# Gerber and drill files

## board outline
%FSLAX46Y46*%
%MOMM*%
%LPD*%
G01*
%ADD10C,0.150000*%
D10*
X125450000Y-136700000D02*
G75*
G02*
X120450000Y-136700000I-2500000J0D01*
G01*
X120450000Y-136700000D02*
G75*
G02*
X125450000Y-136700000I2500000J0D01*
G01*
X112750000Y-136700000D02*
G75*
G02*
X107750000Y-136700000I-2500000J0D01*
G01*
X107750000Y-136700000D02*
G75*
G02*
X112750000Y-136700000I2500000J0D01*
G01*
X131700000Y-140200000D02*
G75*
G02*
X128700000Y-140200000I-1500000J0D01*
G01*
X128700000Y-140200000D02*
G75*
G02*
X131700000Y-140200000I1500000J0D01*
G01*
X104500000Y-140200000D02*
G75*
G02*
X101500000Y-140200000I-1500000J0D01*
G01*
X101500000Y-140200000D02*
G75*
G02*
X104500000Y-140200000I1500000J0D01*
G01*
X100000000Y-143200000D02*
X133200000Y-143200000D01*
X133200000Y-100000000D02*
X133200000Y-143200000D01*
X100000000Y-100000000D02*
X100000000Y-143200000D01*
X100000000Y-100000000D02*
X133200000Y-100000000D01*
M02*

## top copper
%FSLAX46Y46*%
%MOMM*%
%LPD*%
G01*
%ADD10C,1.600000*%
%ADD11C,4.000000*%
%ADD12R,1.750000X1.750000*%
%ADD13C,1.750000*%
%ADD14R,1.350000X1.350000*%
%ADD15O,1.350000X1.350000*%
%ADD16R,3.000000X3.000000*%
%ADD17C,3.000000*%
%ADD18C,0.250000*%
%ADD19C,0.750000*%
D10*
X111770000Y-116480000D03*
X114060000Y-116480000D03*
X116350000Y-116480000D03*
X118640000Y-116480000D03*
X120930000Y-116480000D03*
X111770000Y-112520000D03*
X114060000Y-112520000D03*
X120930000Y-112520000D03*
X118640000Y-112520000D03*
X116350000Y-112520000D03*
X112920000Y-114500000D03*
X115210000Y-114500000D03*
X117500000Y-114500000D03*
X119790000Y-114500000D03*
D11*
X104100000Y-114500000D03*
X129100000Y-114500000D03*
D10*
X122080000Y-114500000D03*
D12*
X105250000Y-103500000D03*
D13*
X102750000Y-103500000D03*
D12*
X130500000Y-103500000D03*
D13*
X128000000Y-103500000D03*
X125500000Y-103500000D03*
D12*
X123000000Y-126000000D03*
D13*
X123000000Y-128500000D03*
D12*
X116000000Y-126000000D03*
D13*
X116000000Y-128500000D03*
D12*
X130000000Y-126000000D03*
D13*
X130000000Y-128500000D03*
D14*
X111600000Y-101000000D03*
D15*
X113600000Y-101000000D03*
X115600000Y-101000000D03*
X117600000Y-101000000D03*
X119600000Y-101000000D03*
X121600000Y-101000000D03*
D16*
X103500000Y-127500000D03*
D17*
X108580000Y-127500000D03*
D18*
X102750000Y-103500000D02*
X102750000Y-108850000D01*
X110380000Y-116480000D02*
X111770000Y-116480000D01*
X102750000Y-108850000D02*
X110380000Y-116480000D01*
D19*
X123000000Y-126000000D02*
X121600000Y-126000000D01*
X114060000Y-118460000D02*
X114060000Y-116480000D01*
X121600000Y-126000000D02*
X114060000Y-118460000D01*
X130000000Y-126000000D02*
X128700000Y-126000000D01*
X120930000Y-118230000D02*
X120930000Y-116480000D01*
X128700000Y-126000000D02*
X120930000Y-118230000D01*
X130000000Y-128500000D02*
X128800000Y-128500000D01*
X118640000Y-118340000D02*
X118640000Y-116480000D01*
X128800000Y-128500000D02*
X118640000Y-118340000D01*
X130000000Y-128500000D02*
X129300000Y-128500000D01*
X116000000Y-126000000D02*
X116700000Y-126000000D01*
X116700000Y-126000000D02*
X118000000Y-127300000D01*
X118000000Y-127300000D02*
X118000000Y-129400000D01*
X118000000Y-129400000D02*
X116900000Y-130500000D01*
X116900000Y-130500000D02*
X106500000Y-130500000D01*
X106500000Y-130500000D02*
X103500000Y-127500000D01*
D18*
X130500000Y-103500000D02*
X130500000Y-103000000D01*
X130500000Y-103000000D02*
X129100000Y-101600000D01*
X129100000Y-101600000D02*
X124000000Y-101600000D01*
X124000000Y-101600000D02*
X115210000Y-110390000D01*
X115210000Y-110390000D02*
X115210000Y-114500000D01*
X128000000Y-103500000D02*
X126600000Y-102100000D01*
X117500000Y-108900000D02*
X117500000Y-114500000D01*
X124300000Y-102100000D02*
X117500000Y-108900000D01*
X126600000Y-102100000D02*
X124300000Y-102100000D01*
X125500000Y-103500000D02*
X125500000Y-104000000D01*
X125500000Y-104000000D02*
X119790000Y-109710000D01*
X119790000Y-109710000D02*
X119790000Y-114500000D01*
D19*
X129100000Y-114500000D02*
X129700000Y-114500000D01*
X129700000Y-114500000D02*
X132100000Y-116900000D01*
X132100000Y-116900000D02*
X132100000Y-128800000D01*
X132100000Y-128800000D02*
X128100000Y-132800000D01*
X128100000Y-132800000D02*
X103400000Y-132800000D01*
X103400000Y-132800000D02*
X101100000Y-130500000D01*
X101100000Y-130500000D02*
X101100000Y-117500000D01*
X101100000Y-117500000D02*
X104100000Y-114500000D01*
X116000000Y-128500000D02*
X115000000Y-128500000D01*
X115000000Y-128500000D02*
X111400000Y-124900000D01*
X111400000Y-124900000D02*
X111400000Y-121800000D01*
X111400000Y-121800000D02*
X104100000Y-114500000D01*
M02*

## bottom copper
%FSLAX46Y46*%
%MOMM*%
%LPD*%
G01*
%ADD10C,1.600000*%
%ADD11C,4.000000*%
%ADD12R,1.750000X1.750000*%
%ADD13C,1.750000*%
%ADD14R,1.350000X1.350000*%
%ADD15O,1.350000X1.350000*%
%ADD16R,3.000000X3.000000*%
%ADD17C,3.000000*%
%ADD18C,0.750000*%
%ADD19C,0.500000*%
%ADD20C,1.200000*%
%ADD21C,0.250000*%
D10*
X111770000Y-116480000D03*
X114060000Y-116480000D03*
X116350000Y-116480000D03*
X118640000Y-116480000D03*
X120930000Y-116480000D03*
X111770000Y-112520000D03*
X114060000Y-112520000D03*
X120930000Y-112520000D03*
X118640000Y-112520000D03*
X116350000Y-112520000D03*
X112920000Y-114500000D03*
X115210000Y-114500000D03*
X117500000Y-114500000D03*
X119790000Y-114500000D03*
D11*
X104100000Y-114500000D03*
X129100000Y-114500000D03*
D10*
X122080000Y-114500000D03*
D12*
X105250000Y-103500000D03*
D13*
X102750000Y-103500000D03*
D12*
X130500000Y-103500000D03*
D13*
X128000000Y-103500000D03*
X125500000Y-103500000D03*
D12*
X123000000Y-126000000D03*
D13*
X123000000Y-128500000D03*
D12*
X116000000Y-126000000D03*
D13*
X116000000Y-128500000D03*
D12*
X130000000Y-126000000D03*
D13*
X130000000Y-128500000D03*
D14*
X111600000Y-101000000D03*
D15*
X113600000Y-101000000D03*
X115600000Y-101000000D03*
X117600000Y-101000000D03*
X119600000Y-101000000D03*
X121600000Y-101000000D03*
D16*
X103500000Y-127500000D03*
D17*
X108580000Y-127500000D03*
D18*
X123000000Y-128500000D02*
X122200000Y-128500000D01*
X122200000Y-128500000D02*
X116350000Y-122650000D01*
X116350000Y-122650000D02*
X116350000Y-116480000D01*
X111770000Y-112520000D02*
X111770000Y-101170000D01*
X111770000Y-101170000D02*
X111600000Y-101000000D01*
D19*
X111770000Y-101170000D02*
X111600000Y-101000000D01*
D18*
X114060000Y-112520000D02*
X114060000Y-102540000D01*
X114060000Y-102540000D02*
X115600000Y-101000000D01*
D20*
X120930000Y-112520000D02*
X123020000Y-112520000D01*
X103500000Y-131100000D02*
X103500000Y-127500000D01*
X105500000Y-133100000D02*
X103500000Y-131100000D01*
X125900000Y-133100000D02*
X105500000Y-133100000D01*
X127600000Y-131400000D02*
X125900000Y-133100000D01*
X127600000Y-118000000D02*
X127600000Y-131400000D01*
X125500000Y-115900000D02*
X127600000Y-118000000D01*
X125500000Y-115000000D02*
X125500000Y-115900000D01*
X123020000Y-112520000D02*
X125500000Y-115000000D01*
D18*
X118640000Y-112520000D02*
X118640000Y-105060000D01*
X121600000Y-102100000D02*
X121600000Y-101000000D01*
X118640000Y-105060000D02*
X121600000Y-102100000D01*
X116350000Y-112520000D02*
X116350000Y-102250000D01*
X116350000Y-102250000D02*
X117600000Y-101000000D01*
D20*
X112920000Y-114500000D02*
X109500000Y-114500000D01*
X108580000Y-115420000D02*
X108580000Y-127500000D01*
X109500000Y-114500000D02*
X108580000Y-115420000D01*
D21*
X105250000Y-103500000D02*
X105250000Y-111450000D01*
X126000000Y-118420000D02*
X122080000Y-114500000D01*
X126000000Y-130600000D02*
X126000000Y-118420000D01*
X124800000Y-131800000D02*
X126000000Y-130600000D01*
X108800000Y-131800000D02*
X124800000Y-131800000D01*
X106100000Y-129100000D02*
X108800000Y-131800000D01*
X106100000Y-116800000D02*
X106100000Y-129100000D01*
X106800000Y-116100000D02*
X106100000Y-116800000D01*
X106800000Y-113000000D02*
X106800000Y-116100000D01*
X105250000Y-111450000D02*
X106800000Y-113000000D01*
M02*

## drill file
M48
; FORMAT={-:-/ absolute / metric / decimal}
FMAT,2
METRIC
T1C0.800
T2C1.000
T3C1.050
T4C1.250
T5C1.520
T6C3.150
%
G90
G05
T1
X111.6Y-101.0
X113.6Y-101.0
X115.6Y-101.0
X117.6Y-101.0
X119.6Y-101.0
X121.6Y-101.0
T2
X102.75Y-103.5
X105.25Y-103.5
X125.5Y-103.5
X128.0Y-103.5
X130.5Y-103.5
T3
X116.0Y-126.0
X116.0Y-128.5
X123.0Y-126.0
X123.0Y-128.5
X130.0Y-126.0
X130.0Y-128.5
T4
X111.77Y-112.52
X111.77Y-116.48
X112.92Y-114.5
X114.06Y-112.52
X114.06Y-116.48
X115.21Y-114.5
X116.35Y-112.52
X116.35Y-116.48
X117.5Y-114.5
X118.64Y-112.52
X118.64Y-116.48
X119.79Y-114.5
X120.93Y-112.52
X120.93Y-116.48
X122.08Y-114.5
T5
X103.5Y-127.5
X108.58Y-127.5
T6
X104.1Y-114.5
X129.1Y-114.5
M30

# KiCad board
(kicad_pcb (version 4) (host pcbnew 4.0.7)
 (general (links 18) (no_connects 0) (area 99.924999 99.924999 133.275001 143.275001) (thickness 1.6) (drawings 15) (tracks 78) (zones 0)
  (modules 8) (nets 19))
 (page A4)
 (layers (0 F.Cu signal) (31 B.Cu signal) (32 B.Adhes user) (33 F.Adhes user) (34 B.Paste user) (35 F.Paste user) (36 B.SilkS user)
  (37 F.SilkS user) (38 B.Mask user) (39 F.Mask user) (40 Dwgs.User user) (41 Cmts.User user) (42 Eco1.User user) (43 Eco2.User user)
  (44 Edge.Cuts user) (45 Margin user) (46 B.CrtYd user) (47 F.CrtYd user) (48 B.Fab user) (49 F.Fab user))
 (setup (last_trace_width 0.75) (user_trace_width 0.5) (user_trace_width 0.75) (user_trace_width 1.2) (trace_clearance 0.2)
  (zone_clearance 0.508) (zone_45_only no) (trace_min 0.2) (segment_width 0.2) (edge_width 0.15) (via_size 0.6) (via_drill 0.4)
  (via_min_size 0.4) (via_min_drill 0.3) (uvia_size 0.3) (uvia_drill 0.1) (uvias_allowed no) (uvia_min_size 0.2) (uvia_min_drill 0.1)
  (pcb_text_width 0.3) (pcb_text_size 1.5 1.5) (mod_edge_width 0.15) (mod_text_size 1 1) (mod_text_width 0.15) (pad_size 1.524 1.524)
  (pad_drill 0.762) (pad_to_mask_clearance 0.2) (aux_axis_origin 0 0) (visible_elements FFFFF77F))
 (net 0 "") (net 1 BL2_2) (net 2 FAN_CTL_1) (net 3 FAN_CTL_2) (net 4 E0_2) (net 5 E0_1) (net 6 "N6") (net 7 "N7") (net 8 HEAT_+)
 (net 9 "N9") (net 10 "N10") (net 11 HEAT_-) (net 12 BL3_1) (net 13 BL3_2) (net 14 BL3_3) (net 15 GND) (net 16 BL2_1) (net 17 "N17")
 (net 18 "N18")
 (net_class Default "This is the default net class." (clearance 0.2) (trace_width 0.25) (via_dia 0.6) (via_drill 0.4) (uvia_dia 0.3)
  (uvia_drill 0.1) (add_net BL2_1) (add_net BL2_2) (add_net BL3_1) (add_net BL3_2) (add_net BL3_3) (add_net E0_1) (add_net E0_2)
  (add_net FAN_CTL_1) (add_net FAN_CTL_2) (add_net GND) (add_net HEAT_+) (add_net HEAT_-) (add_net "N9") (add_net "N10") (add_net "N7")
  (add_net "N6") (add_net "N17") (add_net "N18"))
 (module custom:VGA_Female (layer F.Cu) (at 116.6 114.5)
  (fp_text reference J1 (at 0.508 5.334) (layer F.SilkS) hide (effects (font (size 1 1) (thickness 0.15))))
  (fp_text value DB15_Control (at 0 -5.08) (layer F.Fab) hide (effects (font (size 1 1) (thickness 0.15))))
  (pad 15 thru_hole circle (at -4.83 1.98) (size 1.6 1.6) (drill 1.25) (layers *.Cu *.Mask) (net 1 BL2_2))
  (pad 14 thru_hole circle (at -2.54 1.98) (size 1.6 1.6) (drill 1.25) (layers *.Cu *.Mask) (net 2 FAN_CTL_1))
  (pad 13 thru_hole circle (at -0.25 1.98) (size 1.6 1.6) (drill 1.25) (layers *.Cu *.Mask) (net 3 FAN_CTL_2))
  (pad 12 thru_hole circle (at 2.04 1.98) (size 1.6 1.6) (drill 1.25) (layers *.Cu *.Mask) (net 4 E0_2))
  (pad 11 thru_hole circle (at 4.33 1.98) (size 1.6 1.6) (drill 1.25) (layers *.Cu *.Mask) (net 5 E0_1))
  (pad 5 thru_hole circle (at -4.83 -1.98) (size 1.6 1.6) (drill 1.25) (layers *.Cu *.Mask) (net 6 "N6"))
  (pad 4 thru_hole circle (at -2.54 -1.98) (size 1.6 1.6) (drill 1.25) (layers *.Cu *.Mask) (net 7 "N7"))
  (pad 1 thru_hole circle (at 4.33 -1.98) (size 1.6 1.6) (drill 1.25) (layers *.Cu *.Mask) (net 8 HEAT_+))
  (pad 2 thru_hole circle (at 2.04 -1.98) (size 1.6 1.6) (drill 1.25) (layers *.Cu *.Mask) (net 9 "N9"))
  (pad 3 thru_hole circle (at -0.25 -1.98) (size 1.6 1.6) (drill 1.25) (layers *.Cu *.Mask) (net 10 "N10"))
  (pad 10 thru_hole circle (at -3.68 0) (size 1.6 1.6) (drill 1.25) (layers *.Cu *.Mask) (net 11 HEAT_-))
  (pad 9 thru_hole circle (at -1.39 0) (size 1.6 1.6) (drill 1.25) (layers *.Cu *.Mask) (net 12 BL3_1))
  (pad 8 thru_hole circle (at 0.9 0) (size 1.6 1.6) (drill 1.25) (layers *.Cu *.Mask) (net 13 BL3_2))
  (pad 7 thru_hole circle (at 3.19 0) (size 1.6 1.6) (drill 1.25) (layers *.Cu *.Mask) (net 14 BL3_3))
  (pad 0 thru_hole circle (at -12.5 0) (size 4 4) (drill 3.15) (layers *.Cu *.Mask) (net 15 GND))
  (pad 0 thru_hole circle (at 12.5 0) (size 4 4) (drill 3.15) (layers *.Cu *.Mask) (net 15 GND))
  (pad 6 thru_hole circle (at 5.48 0) (size 1.6 1.6) (drill 1.25) (layers *.Cu *.Mask) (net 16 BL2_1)))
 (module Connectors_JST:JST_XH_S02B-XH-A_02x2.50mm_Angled (layer F.Cu) (at 105.25 103.5 180)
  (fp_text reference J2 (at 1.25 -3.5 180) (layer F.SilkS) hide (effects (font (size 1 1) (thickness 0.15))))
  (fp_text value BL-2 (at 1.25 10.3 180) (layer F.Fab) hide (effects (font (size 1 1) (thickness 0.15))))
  (pad 1 thru_hole rect (at 0 0 180) (size 1.75 1.75) (drill 1) (layers *.Cu *.Mask F.SilkS) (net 16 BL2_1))
  (pad 2 thru_hole circle (at 2.5 0 180) (size 1.75 1.75) (drill 1) (layers *.Cu *.Mask F.SilkS) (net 1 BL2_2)))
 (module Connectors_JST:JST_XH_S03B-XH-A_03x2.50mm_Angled (layer F.Cu) (at 130.5 103.5 180)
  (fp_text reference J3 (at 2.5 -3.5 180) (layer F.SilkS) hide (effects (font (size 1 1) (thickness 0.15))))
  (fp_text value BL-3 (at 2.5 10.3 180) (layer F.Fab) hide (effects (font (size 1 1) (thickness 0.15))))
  (pad 1 thru_hole rect (at 0 0 180) (size 1.75 1.75) (drill 1) (layers *.Cu *.Mask F.SilkS) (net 12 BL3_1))
  (pad 2 thru_hole circle (at 2.5 0 180) (size 1.75 1.75) (drill 1) (layers *.Cu *.Mask F.SilkS) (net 13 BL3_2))
  (pad 3 thru_hole circle (at 5 0 180) (size 1.75 1.75) (drill 1) (layers *.Cu *.Mask F.SilkS) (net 14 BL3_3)))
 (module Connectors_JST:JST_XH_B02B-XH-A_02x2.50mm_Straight (layer F.Cu) (at 123 126 270)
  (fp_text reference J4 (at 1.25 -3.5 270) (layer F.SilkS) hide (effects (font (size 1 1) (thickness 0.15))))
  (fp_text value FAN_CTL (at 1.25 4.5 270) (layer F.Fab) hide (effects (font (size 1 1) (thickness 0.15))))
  (pad 1 thru_hole rect (at 0 0 270) (size 1.75 1.75) (drill 1.05) (layers *.Cu *.Mask) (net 2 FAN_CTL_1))
  (pad 2 thru_hole circle (at 2.5 0 270) (size 1.75 1.75) (drill 1.05) (layers *.Cu *.Mask) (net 3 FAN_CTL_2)))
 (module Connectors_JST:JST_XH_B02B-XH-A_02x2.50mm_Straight (layer F.Cu) (at 116 126 270)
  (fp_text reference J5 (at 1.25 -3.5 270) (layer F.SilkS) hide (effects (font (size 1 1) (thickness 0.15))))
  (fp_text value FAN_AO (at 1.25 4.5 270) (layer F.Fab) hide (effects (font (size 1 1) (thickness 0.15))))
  (pad 1 thru_hole rect (at 0 0 270) (size 1.75 1.75) (drill 1.05) (layers *.Cu *.Mask) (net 8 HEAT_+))
  (pad 2 thru_hole circle (at 2.5 0 270) (size 1.75 1.75) (drill 1.05) (layers *.Cu *.Mask) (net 15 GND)))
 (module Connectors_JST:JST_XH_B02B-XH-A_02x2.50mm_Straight (layer F.Cu) (at 130 126 270)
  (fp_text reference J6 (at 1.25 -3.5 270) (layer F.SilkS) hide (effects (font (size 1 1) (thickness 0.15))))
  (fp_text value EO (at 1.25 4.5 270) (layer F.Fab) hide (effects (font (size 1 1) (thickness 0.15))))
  (pad 1 thru_hole rect (at 0 0 270) (size 1.75 1.75) (drill 1.05) (layers *.Cu *.Mask) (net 5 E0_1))
  (pad 2 thru_hole circle (at 2.5 0 270) (size 1.75 1.75) (drill 1.05) (layers *.Cu *.Mask) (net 4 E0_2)))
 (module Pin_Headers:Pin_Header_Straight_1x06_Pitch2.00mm (layer F.Cu) (at 111.6 101 90)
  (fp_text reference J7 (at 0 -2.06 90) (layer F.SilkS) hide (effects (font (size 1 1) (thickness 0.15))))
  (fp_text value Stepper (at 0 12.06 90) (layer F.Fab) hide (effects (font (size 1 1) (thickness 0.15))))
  (pad 1 thru_hole rect (at 0 0 90) (size 1.35 1.35) (drill 0.8) (layers *.Cu *.Mask) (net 6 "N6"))
  (pad 2 thru_hole oval (at 0 2 90) (size 1.35 1.35) (drill 0.8) (layers *.Cu *.Mask) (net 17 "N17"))
  (pad 3 thru_hole oval (at 0 4 90) (size 1.35 1.35) (drill 0.8) (layers *.Cu *.Mask) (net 7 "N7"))
  (pad 4 thru_hole oval (at 0 6 90) (size 1.35 1.35) (drill 0.8) (layers *.Cu *.Mask) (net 10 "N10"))
  (pad 5 thru_hole oval (at 0 8 90) (size 1.35 1.35) (drill 0.8) (layers *.Cu *.Mask) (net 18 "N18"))
  (pad 6 thru_hole oval (at 0 10 90) (size 1.35 1.35) (drill 0.8) (layers *.Cu *.Mask) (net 9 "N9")))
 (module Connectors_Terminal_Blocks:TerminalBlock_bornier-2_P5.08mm (layer F.Cu) (at 103.5 127.5)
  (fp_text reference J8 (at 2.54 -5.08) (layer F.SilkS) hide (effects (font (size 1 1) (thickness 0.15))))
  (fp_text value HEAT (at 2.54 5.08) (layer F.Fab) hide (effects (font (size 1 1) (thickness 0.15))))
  (pad 1 thru_hole rect (at 0 0) (size 3 3) (drill 1.52) (layers *.Cu *.Mask) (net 8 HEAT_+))
  (pad 2 thru_hole circle (at 5.08 0) (size 3 3) (drill 1.52) (layers *.Cu *.Mask) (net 11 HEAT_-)))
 (gr_circle (center 122.95 136.7) (end 125.45 136.7) (layer Edge.Cuts) (width 0.15))
 (gr_circle (center 110.25 136.7) (end 112.75 136.7) (layer Edge.Cuts) (width 0.15))
 (gr_circle (center 130.2 140.2) (end 131.7 140.2) (layer Edge.Cuts) (width 0.15))
 (gr_circle (center 103 140.2) (end 104.5 140.2) (layer Edge.Cuts) (width 0.15))
 (gr_line (start 100 143.2) (end 133.2 143.2) (angle 90) (layer Edge.Cuts) (width 0.15))
 (gr_line (start 133.2 100) (end 133.2 143.2) (angle 90) (layer Edge.Cuts) (width 0.15))
 (gr_line (start 100 100) (end 100 143.2) (angle 90) (layer Edge.Cuts) (width 0.15))
 (gr_line (start 100 100) (end 133.2 100) (angle 90) (layer Edge.Cuts) (width 0.15))
 (segment (start 102.75 103.5) (end 102.75 108.85) (width 0.25) (layer F.Cu) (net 1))
 (segment (start 110.38 116.48) (end 111.77 116.48) (width 0.25) (layer F.Cu) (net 1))
 (segment (start 102.75 108.85) (end 110.38 116.48) (width 0.25) (layer F.Cu) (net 1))
 (segment (start 123 128.5) (end 122.2 128.5) (width 0.75) (layer B.Cu) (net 3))
 (segment (start 122.2 128.5) (end 116.35 122.65) (width 0.75) (layer B.Cu) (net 3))
 (segment (start 116.35 122.65) (end 116.35 116.48) (width 0.75) (layer B.Cu) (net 3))
 (segment (start 123 126) (end 121.6 126) (width 0.75) (layer F.Cu) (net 2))
 (segment (start 114.06 118.46) (end 114.06 116.48) (width 0.75) (layer F.Cu) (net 2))
 (segment (start 121.6 126) (end 114.06 118.46) (width 0.75) (layer F.Cu) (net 2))
 (segment (start 130 126) (end 128.7 126) (width 0.75) (layer F.Cu) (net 5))
 (segment (start 120.93 118.23) (end 120.93 116.48) (width 0.75) (layer F.Cu) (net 5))
 (segment (start 128.7 126) (end 120.93 118.23) (width 0.75) (layer F.Cu) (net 5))
 (segment (start 130 128.5) (end 128.8 128.5) (width 0.75) (layer F.Cu) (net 4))
 (segment (start 118.64 118.34) (end 118.64 116.48) (width 0.75) (layer F.Cu) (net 4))
 (segment (start 128.8 128.5) (end 118.64 118.34) (width 0.75) (layer F.Cu) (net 4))
 (segment (start 130 128.5) (end 129.3 128.5) (width 0.75) (layer F.Cu) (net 4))
 (segment (start 111.77 112.52) (end 111.77 101.17) (width 0.75) (layer B.Cu) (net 6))
 (segment (start 111.77 101.17) (end 111.6 101) (width 0.75) (layer B.Cu) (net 6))
 (segment (start 111.77 101.17) (end 111.6 101) (width 0.5) (layer B.Cu) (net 6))
 (segment (start 114.06 112.52) (end 114.06 102.54) (width 0.75) (layer B.Cu) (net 7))
 (segment (start 114.06 102.54) (end 115.6 101) (width 0.75) (layer B.Cu) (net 7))
 (segment (start 120.93 112.52) (end 123.02 112.52) (width 1.2) (layer B.Cu) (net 8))
 (segment (start 103.5 131.1) (end 103.5 127.5) (width 1.2) (layer B.Cu) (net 8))
 (segment (start 105.5 133.1) (end 103.5 131.1) (width 1.2) (layer B.Cu) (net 8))
 (segment (start 125.9 133.1) (end 105.5 133.1) (width 1.2) (layer B.Cu) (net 8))
 (segment (start 127.6 131.4) (end 125.9 133.1) (width 1.2) (layer B.Cu) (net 8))
 (segment (start 127.6 118) (end 127.6 131.4) (width 1.2) (layer B.Cu) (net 8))
 (segment (start 125.5 115.9) (end 127.6 118) (width 1.2) (layer B.Cu) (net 8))
 (segment (start 125.5 115) (end 125.5 115.9) (width 1.2) (layer B.Cu) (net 8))
 (segment (start 123.02 112.52) (end 125.5 115) (width 1.2) (layer B.Cu) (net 8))
 (segment (start 116 126) (end 116.7 126) (width 0.75) (layer F.Cu) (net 8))
 (segment (start 116.7 126) (end 118 127.3) (width 0.75) (layer F.Cu) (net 8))
 (segment (start 118 127.3) (end 118 129.4) (width 0.75) (layer F.Cu) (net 8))
 (segment (start 118 129.4) (end 116.9 130.5) (width 0.75) (layer F.Cu) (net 8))
 (segment (start 116.9 130.5) (end 106.5 130.5) (width 0.75) (layer F.Cu) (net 8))
 (segment (start 106.5 130.5) (end 103.5 127.5) (width 0.75) (layer F.Cu) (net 8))
 (segment (start 118.64 112.52) (end 118.64 105.06) (width 0.75) (layer B.Cu) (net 9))
 (segment (start 121.6 102.1) (end 121.6 101) (width 0.75) (layer B.Cu) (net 9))
 (segment (start 118.64 105.06) (end 121.6 102.1) (width 0.75) (layer B.Cu) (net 9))
 (segment (start 116.35 112.52) (end 116.35 102.25) (width 0.75) (layer B.Cu) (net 10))
 (segment (start 116.35 102.25) (end 117.6 101) (width 0.75) (layer B.Cu) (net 10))
 (segment (start 112.92 114.5) (end 109.5 114.5) (width 1.2) (layer B.Cu) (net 11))
 (segment (start 108.58 115.42) (end 108.58 127.5) (width 1.2) (layer B.Cu) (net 11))
 (segment (start 109.5 114.5) (end 108.58 115.42) (width 1.2) (layer B.Cu) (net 11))
 (segment (start 130.5 103.5) (end 130.5 103) (width 0.25) (layer F.Cu) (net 12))
 (segment (start 130.5 103) (end 129.1 101.6) (width 0.25) (layer F.Cu) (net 12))
 (segment (start 129.1 101.6) (end 124 101.6) (width 0.25) (layer F.Cu) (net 12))
 (segment (start 124 101.6) (end 115.21 110.39) (width 0.25) (layer F.Cu) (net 12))
 (segment (start 115.21 110.39) (end 115.21 114.5) (width 0.25) (layer F.Cu) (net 12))
 (segment (start 128 103.5) (end 126.6 102.1) (width 0.25) (layer F.Cu) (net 13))
 (segment (start 117.5 108.9) (end 117.5 114.5) (width 0.25) (layer F.Cu) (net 13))
 (segment (start 124.3 102.1) (end 117.5 108.9) (width 0.25) (layer F.Cu) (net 13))
 (segment (start 126.6 102.1) (end 124.3 102.1) (width 0.25) (layer F.Cu) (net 13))
 (segment (start 125.5 103.5) (end 125.5 104) (width 0.25) (layer F.Cu) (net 14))
 (segment (start 125.5 104) (end 119.79 109.71) (width 0.25) (layer F.Cu) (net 14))
 (segment (start 119.79 109.71) (end 119.79 114.5) (width 0.25) (layer F.Cu) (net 14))
 (segment (start 129.1 114.5) (end 129.7 114.5) (width 0.75) (layer F.Cu) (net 15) (status C00000))
 (segment (start 129.7 114.5) (end 132.1 116.9) (width 0.75) (layer F.Cu) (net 15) (status 400000))
 (segment (start 132.1 116.9) (end 132.1 128.8) (width 0.75) (layer F.Cu) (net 15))
 (segment (start 132.1 128.8) (end 128.1 132.8) (width 0.75) (layer F.Cu) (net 15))
 (segment (start 128.1 132.8) (end 103.4 132.8) (width 0.75) (layer F.Cu) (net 15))
 (segment (start 103.4 132.8) (end 101.1 130.5) (width 0.75) (layer F.Cu) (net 15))
 (segment (start 101.1 130.5) (end 101.1 117.5) (width 0.75) (layer F.Cu) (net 15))
 (segment (start 101.1 117.5) (end 104.1 114.5) (width 0.75) (layer F.Cu) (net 15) (status 800000))
 (segment (start 116 128.5) (end 115 128.5) (width 0.75) (layer F.Cu) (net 15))
 (segment (start 115 128.5) (end 111.4 124.9) (width 0.75) (layer F.Cu) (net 15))
 (segment (start 111.4 124.9) (end 111.4 121.8) (width 0.75) (layer F.Cu) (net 15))
 (segment (start 111.4 121.8) (end 104.1 114.5) (width 0.75) (layer F.Cu) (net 15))
 (segment (start 105.25 103.5) (end 105.25 111.45) (width 0.25) (layer B.Cu) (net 16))
 (segment (start 126 118.42) (end 122.08 114.5) (width 0.25) (layer B.Cu) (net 16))
 (segment (start 126 130.6) (end 126 118.42) (width 0.25) (layer B.Cu) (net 16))
 (segment (start 124.8 131.8) (end 126 130.6) (width 0.25) (layer B.Cu) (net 16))
 (segment (start 108.8 131.8) (end 124.8 131.8) (width 0.25) (layer B.Cu) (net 16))
 (segment (start 106.1 129.1) (end 108.8 131.8) (width 0.25) (layer B.Cu) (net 16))
 (segment (start 106.1 116.8) (end 106.1 129.1) (width 0.25) (layer B.Cu) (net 16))
 (segment (start 106.8 116.1) (end 106.1 116.8) (width 0.25) (layer B.Cu) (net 16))
 (segment (start 106.8 113) (end 106.8 116.1) (width 0.25) (layer B.Cu) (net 16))
 (segment (start 105.25 111.45) (end 106.8 113) (width 0.25) (layer B.Cu) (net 16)))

